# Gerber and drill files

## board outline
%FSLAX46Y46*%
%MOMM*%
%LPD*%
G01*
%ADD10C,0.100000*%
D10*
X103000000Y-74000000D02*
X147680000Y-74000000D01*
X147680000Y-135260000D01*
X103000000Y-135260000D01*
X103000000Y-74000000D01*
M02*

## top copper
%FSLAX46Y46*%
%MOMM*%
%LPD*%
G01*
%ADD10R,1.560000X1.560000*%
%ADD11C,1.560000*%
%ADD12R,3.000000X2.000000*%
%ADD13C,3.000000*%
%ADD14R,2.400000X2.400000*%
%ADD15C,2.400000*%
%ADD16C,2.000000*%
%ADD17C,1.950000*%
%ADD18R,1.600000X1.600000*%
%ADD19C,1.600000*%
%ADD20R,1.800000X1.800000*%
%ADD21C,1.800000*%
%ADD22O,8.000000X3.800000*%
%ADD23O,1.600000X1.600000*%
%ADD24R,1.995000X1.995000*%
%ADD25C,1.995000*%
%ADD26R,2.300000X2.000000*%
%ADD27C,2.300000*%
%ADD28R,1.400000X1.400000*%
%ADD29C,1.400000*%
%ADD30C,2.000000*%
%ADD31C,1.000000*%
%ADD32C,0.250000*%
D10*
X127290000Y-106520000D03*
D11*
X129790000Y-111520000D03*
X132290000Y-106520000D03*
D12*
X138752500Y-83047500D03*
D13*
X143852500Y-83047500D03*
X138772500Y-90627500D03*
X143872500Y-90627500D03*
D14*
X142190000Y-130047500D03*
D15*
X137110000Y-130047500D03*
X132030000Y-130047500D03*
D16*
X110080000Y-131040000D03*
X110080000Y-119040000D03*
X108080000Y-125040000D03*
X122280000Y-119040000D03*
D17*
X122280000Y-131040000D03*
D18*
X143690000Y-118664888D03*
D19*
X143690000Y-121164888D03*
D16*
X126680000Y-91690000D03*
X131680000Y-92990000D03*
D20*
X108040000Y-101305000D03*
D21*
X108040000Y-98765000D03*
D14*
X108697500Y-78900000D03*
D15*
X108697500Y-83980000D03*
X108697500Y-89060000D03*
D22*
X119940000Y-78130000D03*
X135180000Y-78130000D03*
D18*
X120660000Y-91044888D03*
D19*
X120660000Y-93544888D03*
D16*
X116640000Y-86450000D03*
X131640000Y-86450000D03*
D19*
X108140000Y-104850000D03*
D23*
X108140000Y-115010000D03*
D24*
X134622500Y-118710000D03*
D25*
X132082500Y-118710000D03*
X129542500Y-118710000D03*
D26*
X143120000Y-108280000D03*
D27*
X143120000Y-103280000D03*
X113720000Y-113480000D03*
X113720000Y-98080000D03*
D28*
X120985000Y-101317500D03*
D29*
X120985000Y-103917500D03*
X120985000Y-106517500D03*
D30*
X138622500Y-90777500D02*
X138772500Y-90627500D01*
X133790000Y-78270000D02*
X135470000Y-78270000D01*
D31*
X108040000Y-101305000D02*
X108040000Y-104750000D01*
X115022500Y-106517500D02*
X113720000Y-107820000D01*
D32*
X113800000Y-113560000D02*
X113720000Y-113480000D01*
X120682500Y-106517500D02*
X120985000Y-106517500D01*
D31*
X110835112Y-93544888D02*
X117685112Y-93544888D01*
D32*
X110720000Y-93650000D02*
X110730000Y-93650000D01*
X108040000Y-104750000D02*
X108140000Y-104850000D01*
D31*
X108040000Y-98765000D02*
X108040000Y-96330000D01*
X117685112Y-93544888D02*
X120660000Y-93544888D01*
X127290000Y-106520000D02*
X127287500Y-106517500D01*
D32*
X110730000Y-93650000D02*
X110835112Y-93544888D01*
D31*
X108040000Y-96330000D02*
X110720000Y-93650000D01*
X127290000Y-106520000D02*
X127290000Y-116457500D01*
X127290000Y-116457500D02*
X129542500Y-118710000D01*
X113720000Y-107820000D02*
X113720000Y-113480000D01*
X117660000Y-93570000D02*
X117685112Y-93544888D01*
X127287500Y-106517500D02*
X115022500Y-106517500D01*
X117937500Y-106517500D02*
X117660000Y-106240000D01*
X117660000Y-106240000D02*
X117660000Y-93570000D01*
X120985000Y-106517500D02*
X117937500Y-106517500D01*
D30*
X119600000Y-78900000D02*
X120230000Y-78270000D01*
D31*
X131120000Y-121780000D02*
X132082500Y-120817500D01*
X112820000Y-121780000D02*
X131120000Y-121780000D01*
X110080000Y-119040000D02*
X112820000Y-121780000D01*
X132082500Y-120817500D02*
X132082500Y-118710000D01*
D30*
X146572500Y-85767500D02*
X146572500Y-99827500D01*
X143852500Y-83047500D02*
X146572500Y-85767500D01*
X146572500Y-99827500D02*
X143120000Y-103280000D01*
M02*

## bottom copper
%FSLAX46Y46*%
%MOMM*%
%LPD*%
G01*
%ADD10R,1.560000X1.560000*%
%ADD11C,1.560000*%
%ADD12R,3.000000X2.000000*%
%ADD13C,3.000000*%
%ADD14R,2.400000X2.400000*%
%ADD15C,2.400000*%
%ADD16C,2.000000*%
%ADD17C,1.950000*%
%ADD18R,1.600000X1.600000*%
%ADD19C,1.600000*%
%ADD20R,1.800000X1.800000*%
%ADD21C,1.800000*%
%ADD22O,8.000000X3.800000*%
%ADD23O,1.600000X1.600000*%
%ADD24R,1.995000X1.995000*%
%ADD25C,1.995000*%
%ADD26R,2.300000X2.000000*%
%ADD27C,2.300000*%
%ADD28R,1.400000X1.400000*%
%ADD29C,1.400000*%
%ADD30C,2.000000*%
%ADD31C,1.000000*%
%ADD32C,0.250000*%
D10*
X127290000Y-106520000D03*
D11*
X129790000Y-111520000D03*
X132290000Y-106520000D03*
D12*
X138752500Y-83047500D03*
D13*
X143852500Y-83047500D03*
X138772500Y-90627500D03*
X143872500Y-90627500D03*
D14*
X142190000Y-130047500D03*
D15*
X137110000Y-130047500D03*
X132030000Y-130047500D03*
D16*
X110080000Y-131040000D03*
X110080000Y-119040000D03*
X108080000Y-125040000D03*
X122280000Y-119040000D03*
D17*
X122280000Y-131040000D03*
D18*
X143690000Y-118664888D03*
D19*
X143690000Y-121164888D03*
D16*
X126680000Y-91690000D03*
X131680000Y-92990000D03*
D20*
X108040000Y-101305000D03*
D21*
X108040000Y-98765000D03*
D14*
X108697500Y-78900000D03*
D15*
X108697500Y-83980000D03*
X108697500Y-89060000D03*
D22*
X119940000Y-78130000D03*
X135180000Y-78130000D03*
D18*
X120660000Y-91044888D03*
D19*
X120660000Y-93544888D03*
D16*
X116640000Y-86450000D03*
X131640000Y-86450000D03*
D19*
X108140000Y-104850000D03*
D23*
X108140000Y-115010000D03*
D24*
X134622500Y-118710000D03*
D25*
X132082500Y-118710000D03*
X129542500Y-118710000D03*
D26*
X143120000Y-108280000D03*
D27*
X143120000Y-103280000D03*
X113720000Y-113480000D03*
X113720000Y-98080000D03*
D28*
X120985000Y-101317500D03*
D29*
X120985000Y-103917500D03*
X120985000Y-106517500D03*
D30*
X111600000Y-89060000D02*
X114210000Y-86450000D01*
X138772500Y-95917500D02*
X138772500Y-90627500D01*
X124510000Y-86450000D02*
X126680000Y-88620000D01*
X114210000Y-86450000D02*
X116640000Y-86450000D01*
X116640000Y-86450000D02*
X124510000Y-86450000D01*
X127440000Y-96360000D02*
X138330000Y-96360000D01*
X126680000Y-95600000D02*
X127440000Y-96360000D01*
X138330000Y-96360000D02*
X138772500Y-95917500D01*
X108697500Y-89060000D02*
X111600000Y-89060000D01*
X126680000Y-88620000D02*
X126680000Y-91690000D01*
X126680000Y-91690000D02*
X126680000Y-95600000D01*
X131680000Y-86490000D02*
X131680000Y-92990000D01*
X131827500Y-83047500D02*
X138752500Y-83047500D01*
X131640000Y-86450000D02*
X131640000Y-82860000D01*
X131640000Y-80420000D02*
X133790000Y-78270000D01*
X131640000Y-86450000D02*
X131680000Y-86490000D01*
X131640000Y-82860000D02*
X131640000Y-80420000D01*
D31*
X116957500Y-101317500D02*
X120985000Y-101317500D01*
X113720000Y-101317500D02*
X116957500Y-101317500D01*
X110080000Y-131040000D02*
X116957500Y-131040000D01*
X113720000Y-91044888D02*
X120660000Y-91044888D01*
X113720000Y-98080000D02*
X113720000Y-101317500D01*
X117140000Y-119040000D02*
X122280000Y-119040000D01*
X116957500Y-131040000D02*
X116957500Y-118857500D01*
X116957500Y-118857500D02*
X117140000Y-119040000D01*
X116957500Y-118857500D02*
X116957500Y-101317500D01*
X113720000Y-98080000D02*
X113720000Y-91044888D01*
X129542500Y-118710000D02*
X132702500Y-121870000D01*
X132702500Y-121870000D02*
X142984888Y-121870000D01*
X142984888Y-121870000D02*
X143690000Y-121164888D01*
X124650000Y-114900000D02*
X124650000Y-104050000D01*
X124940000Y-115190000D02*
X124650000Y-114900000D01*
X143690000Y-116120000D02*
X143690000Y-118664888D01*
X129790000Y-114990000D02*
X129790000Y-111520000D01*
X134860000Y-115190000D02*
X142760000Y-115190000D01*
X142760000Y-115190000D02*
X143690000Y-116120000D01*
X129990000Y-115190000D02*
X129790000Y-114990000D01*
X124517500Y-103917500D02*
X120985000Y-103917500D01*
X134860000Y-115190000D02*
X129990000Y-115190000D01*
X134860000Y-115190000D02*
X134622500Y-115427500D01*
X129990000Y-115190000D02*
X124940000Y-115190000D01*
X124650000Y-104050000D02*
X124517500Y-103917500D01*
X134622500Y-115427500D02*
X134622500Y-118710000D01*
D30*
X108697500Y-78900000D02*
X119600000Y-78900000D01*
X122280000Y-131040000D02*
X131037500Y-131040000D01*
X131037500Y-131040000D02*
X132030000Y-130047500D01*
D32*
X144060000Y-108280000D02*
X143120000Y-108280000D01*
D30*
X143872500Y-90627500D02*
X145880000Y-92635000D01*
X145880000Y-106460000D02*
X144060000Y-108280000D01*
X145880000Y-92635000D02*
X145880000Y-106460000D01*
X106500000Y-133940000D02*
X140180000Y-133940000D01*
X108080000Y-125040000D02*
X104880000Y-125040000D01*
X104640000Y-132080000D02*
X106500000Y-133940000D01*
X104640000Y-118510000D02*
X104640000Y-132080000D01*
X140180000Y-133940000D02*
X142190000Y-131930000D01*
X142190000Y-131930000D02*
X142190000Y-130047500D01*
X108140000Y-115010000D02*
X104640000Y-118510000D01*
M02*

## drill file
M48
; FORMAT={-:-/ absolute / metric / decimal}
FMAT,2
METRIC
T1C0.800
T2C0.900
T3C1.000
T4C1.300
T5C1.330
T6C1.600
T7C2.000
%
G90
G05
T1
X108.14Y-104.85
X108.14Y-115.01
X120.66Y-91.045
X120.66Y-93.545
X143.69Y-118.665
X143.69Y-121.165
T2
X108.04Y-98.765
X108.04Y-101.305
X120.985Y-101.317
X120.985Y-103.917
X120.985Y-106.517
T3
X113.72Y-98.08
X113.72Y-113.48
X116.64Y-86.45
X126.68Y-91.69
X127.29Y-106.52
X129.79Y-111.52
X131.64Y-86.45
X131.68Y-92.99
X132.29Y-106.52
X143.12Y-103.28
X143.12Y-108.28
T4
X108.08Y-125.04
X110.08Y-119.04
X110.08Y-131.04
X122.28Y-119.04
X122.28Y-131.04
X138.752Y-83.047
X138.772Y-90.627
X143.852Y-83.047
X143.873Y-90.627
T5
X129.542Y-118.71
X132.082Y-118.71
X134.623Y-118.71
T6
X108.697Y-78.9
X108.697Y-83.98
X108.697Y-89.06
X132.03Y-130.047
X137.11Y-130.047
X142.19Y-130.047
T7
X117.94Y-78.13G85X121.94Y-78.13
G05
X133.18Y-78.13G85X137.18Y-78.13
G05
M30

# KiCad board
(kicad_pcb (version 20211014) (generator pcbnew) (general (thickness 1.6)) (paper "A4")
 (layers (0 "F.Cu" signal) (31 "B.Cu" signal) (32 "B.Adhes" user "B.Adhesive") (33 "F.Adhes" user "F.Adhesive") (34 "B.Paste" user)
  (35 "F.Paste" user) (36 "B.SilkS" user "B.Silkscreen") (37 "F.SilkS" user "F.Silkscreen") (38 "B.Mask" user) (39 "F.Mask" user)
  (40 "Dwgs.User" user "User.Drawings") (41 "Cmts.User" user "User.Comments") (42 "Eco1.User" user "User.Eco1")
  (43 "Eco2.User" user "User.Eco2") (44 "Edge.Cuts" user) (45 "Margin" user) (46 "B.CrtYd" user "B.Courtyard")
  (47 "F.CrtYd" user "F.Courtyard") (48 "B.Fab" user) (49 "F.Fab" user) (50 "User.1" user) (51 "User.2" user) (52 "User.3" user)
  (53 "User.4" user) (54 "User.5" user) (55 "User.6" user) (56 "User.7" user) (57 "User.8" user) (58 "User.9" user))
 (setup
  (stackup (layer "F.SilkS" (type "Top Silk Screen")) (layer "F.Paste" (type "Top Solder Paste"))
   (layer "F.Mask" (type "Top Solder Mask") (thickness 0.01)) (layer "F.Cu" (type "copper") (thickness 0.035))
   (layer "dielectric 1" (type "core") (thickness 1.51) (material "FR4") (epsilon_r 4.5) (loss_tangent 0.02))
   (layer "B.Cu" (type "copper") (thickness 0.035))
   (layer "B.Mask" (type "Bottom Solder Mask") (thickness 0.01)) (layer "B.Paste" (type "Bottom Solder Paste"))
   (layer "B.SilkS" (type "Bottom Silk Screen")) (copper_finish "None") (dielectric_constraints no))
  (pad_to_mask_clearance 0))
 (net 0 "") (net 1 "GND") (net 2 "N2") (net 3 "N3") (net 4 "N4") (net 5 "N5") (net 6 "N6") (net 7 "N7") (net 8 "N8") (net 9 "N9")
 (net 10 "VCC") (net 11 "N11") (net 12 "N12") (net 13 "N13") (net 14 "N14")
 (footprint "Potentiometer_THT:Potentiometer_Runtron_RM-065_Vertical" (layer "F.Cu") (at 127.29 106.52)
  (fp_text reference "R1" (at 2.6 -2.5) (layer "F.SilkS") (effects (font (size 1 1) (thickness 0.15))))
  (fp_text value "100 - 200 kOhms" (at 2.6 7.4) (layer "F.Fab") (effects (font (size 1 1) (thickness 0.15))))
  (pad "1" thru_hole rect (at 0 0) (size 1.56 1.56) (drill 1) (layers *.Cu *.Mask) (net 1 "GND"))
  (pad "2" thru_hole circle (at 2.5 5) (size 1.56 1.56) (drill 1) (layers *.Cu *.Mask) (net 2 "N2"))
  (pad "3" thru_hole circle (at 5 0) (size 1.56 1.56) (drill 1) (layers *.Cu *.Mask)))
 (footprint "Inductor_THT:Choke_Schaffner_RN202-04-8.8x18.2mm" (layer "F.Cu") (at 138.7725 75.4275)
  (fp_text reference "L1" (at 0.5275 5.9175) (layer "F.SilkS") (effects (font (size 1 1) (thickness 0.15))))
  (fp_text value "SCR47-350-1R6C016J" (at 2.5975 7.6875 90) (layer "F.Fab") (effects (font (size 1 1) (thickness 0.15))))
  (pad "1" thru_hole rect (at -0.02 7.62) (size 3 2) (drill 1.3) (layers *.Cu *.Mask) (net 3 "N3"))
  (pad "2" thru_hole circle (at 5.08 7.62) (size 3 3) (drill 1.3) (layers *.Cu *.Mask) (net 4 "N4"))
  (pad "3" thru_hole circle (at 0 15.2) (size 3 3) (drill 1.3) (layers *.Cu *.Mask) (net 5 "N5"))
  (pad "4" thru_hole circle (at 5.1 15.2) (size 3 3) (drill 1.3) (layers *.Cu *.Mask) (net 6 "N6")))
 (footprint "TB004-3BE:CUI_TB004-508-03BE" (layer "F.Cu") (at 142.19 130.0475 180)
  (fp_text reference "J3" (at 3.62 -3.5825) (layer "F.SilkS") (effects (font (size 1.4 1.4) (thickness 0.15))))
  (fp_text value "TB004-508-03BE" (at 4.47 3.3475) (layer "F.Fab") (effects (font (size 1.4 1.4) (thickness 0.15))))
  (pad "1" thru_hole rect locked (at 0 0 180) (size 2.4 2.4) (drill 1.6) (layers *.Cu *.Mask) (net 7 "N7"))
  (pad "2" thru_hole circle locked (at 5.08 0 180) (size 2.4 2.4) (drill 1.6) (layers *.Cu *.Mask) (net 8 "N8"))
  (pad "3" thru_hole circle locked (at 10.16 0 180) (size 2.4 2.4) (drill 1.6) (layers *.Cu *.Mask) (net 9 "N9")))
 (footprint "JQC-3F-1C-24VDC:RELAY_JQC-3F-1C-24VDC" (layer "F.Cu") (at 116.18 125.04 180)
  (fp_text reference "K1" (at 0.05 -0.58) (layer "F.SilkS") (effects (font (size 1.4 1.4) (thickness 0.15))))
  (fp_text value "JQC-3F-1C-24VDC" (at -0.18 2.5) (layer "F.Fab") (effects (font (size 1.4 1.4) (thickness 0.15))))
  (pad "COIL1" thru_hole circle locked (at 6.1 -6 180) (size 2 2) (drill 1.3) (layers *.Cu *.Mask) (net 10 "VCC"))
  (pad "COIL2" thru_hole circle locked (at 6.1 6 180) (size 2 2) (drill 1.3) (layers *.Cu *.Mask) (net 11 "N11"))
  (pad "COM" thru_hole circle locked (at 8.1 0 180) (size 2 2) (drill 1.3) (layers *.Cu *.Mask) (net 7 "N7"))
  (pad "NC" thru_hole circle locked (at -6.1 6 180) (size 2 2) (drill 1.3) (layers *.Cu *.Mask) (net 10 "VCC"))
  (pad "NO" thru_hole circle locked (at -6.1 -6 180) (size 1.95 1.95) (drill 1.3) (layers *.Cu *.Mask) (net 9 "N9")))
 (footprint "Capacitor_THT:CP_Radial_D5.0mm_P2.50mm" (layer "F.Cu") (at 143.69 118.664888 -90)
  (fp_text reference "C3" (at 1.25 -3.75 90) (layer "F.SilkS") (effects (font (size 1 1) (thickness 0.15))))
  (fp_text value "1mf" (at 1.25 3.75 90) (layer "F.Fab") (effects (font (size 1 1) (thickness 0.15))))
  (pad "1" thru_hole rect (at 0 0 270) (size 1.6 1.6) (drill 0.8) (layers *.Cu *.Mask) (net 2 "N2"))
  (pad "2" thru_hole circle (at 2.5 0 270) (size 1.6 1.6) (drill 0.8) (layers *.Cu *.Mask) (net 1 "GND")))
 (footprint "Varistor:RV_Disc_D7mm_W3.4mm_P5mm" (layer "F.Cu") (at 126.68 91.69)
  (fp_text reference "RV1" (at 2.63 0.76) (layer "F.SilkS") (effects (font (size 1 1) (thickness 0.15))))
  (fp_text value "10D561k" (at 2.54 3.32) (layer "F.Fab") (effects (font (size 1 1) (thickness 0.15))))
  (pad "1" thru_hole circle (at 0 0) (size 2 2) (drill 1) (layers *.Cu *.Mask) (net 5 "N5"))
  (pad "2" thru_hole circle (at 5 1.3) (size 2 2) (drill 1) (layers *.Cu *.Mask "F.Adhes") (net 3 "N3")))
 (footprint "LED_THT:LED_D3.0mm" (layer "F.Cu") (at 108.04 101.305 90)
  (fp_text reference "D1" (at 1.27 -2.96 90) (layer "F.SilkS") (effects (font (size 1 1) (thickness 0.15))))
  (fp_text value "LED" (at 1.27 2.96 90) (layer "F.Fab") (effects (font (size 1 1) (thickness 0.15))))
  (pad "1" thru_hole rect (at 0 0 90) (size 1.8 1.8) (drill 0.9) (layers *.Cu *.Mask) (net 1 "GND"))
  (pad "2" thru_hole circle (at 2.54 0 90) (size 1.8 1.8) (drill 0.9) (layers *.Cu *.Mask) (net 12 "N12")))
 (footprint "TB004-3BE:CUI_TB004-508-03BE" (layer "F.Cu") (at 108.6975 78.9 -90)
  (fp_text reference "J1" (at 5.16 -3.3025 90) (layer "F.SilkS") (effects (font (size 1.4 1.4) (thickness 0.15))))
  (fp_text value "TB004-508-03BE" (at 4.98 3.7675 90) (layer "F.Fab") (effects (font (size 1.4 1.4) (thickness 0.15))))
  (pad "1" thru_hole rect locked (at 0 0 270) (size 2.4 2.4) (drill 1.6) (layers *.Cu *.Mask) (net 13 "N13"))
  (pad "2" thru_hole circle locked (at 5.08 0 270) (size 2.4 2.4) (drill 1.6) (layers *.Cu *.Mask) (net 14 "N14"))
  (pad "3" thru_hole circle locked (at 10.16 0 270) (size 2.4 2.4) (drill 1.6) (layers *.Cu *.Mask) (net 5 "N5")))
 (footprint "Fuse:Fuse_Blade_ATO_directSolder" (layer "F.Cu") (at 122.48 78.13)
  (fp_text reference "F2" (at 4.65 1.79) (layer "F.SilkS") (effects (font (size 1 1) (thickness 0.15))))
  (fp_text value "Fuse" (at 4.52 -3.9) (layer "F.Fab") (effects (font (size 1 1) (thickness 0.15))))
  (pad "1" thru_hole oval (at -2.54 0) (size 8 3.8) (drill oval 6 2) (layers *.Cu *.Mask) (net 13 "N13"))
  (pad "2" thru_hole oval (at 12.7 0) (size 8 3.8) (drill oval 6 2) (layers *.Cu *.Mask) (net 3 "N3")))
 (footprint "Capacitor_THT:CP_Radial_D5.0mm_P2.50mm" (layer "F.Cu") (at 120.66 91.044888 -90)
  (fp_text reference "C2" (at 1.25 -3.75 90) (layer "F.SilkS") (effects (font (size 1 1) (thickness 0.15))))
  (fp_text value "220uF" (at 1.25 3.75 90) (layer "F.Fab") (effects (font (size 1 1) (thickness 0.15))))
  (pad "1" thru_hole rect (at 0 0 270) (size 1.6 1.6) (drill 0.8) (layers *.Cu *.Mask) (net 10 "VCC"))
  (pad "2" thru_hole circle (at 2.5 0 270) (size 1.6 1.6) (drill 0.8) (layers *.Cu *.Mask) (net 1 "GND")))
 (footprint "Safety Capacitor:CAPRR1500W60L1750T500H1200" (layer "F.Cu") (at 124.14 86.45)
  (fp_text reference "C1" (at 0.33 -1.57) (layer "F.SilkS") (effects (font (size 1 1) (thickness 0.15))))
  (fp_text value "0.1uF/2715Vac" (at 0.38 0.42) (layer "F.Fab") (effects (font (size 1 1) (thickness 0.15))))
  (pad "1" thru_hole circle locked (at -7.5 0) (size 2 2) (drill 1) (layers *.Cu *.Mask) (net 5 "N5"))
  (pad "2" thru_hole circle locked (at 7.5 0) (size 2 2) (drill 1) (layers *.Cu *.Mask) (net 3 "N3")))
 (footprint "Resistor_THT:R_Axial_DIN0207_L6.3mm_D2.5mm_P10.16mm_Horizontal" (layer "F.Cu") (at 108.14 104.85 -90)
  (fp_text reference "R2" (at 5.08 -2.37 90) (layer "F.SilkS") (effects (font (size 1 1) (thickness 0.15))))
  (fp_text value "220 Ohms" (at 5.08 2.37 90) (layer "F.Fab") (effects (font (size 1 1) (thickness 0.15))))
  (pad "1" thru_hole circle (at 0 0 270) (size 1.6 1.6) (drill 0.8) (layers *.Cu *.Mask) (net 12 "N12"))
  (pad "2" thru_hole oval (at 10.16 0 270) (size 1.6 1.6) (drill 0.8) (layers *.Cu *.Mask) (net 7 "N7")))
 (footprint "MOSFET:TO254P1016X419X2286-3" (layer "F.Cu") (at 132.0825 118.71 180)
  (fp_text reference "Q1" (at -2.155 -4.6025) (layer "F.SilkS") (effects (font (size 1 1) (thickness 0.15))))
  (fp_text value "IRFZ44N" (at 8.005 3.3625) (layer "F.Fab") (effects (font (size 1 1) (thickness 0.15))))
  (pad "1" thru_hole rect (at -2.54 0 180) (size 1.995 1.995) (drill 1.33) (layers *.Cu *.Mask) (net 2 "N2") (solder_mask_margin 0.102))
  (pad "2" thru_hole circle (at 0 0 180) (size 1.995 1.995) (drill 1.33) (layers *.Cu *.Mask) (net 11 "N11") (solder_mask_margin 0.102))
  (pad "3" thru_hole circle (at 2.54 0 180) (size 1.995 1.995) (drill 1.33) (layers *.Cu *.Mask) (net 1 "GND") (solder_mask_margin 0.102)))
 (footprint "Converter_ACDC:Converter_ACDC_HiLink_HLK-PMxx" (layer "F.Cu") (at 143.12 108.28 180)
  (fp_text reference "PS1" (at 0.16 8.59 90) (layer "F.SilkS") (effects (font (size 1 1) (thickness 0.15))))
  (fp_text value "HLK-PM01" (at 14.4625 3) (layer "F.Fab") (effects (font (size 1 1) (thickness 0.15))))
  (pad "1" thru_hole rect (at 0 0 180) (size 2.3 2) (drill 1) (layers *.Cu *.Mask) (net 6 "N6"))
  (pad "2" thru_hole circle (at 0 5 180) (size 2.3 2.3) (drill 1) (layers *.Cu *.Mask) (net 4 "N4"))
  (pad "3" thru_hole circle (at 29.4 -5.2 180) (size 2.3 2.3) (drill 1) (layers *.Cu *.Mask) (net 1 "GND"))
  (pad "4" thru_hole circle (at 29.4 10.2 180) (size 2.3 2.3) (drill 1) (layers *.Cu *.Mask) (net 10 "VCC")))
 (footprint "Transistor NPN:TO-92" (layer "B.Cu") (at 120.985 103.9175 -90)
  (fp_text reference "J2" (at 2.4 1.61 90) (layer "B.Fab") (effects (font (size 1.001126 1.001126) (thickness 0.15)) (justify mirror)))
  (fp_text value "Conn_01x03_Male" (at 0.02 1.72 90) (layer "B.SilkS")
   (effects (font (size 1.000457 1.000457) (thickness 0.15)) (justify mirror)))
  (pad "1" thru_hole rect locked (at -2.6 0 270) (size 1.4 1.4) (drill 0.9) (layers *.Cu *.Mask) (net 10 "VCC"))
  (pad "2" thru_hole circle locked (at 0 0 270) (size 1.4 1.4) (drill 0.9) (layers *.Cu *.Mask) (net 2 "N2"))
  (pad "3" thru_hole circle locked (at 2.6 0 270) (size 1.4 1.4) (drill 0.9) (layers *.Cu *.Mask) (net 1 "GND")))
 (gr_rect (start 103 74) (end 147.68 135.26) (layer "Edge.Cuts") (width 0.1) (fill none))
 (segment (start 138.6225 90.7775) (end 138.7725 90.6275) (width 2) (layer "F.Cu") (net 5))
 (segment (start 111.6 89.06) (end 114.21 86.45) (width 2) (layer "B.Cu") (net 5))
 (segment (start 138.7725 95.9175) (end 138.7725 90.6275) (width 2) (layer "B.Cu") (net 5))
 (segment (start 124.51 86.45) (end 126.68 88.62) (width 2) (layer "B.Cu") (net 5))
 (segment (start 114.21 86.45) (end 116.64 86.45) (width 2) (layer "B.Cu") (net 5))
 (segment (start 116.64 86.45) (end 124.51 86.45) (width 2) (layer "B.Cu") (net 5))
 (segment (start 127.44 96.36) (end 138.33 96.36) (width 2) (layer "B.Cu") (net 5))
 (segment (start 126.68 95.6) (end 127.44 96.36) (width 2) (layer "B.Cu") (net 5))
 (segment (start 138.33 96.36) (end 138.7725 95.9175) (width 2) (layer "B.Cu") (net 5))
 (segment (start 108.6975 89.06) (end 111.6 89.06) (width 2) (layer "B.Cu") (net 5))
 (segment (start 126.68 88.62) (end 126.68 91.69) (width 2) (layer "B.Cu") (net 5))
 (segment (start 126.68 91.69) (end 126.68 95.6) (width 2) (layer "B.Cu") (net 5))
 (segment (start 133.79 78.27) (end 135.47 78.27) (width 2) (layer "F.Cu") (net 3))
 (segment (start 131.68 86.49) (end 131.68 92.99) (width 2) (layer "B.Cu") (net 3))
 (segment (start 131.8275 83.0475) (end 138.7525 83.0475) (width 2) (layer "B.Cu") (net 3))
 (segment (start 131.64 86.45) (end 131.64 82.86) (width 2) (layer "B.Cu") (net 3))
 (segment (start 131.64 80.42) (end 133.79 78.27) (width 2) (layer "B.Cu") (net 3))
 (segment (start 131.64 86.45) (end 131.68 86.49) (width 2) (layer "B.Cu") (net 3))
 (segment (start 131.64 82.86) (end 131.64 80.42) (width 2) (layer "B.Cu") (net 3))
 (segment (start 116.9575 101.3175) (end 120.985 101.3175) (width 1) (layer "B.Cu") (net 10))
 (segment (start 113.72 101.3175) (end 116.9575 101.3175) (width 1) (layer "B.Cu") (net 10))
 (segment (start 110.08 131.04) (end 116.9575 131.04) (width 1) (layer "B.Cu") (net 10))
 (segment (start 113.72 91.044888) (end 120.66 91.044888) (width 1) (layer "B.Cu") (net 10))
 (segment (start 113.72 98.08) (end 113.72 101.3175) (width 1) (layer "B.Cu") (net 10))
 (segment (start 117.14 119.04) (end 122.28 119.04) (width 1) (layer "B.Cu") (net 10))
 (segment (start 116.9575 131.04) (end 116.9575 118.8575) (width 1) (layer "B.Cu") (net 10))
 (segment (start 116.9575 118.8575) (end 117.14 119.04) (width 1) (layer "B.Cu") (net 10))
 (segment (start 116.9575 118.8575) (end 116.9575 101.3175) (width 1) (layer "B.Cu") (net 10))
 (segment (start 113.72 98.08) (end 113.72 91.044888) (width 1) (layer "B.Cu") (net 10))
 (segment (start 108.04 101.305) (end 108.04 104.75) (width 1) (layer "F.Cu") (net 1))
 (segment (start 115.0225 106.5175) (end 113.72 107.82) (width 1) (layer "F.Cu") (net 1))
 (segment (start 113.8 113.56) (end 113.72 113.48) (width 0.25) (layer "F.Cu") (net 1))
 (segment (start 120.6825 106.5175) (end 120.985 106.5175) (width 0.25) (layer "F.Cu") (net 1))
 (segment (start 110.835112 93.544888) (end 117.685112 93.544888) (width 1) (layer "F.Cu") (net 1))
 (segment (start 110.72 93.65) (end 110.73 93.65) (width 0.25) (layer "F.Cu") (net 1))
 (segment (start 108.04 104.75) (end 108.14 104.85) (width 0.25) (layer "F.Cu") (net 1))
 (segment (start 108.04 98.765) (end 108.04 96.33) (width 1) (layer "F.Cu") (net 1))
 (segment (start 117.685112 93.544888) (end 120.66 93.544888) (width 1) (layer "F.Cu") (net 1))
 (segment (start 127.29 106.52) (end 127.2875 106.5175) (width 1) (layer "F.Cu") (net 1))
 (segment (start 110.73 93.65) (end 110.835112 93.544888) (width 0.25) (layer "F.Cu") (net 1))
 (segment (start 108.04 96.33) (end 110.72 93.65) (width 1) (layer "F.Cu") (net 1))
 (segment (start 127.29 106.52) (end 127.29 116.4575) (width 1) (layer "F.Cu") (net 1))
 (segment (start 127.29 116.4575) (end 129.5425 118.71) (width 1) (layer "F.Cu") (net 1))
 (segment (start 113.72 107.82) (end 113.72 113.48) (width 1) (layer "F.Cu") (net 1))
 (segment (start 117.66 93.57) (end 117.685112 93.544888) (width 1) (layer "F.Cu") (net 1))
 (segment (start 127.2875 106.5175) (end 115.0225 106.5175) (width 1) (layer "F.Cu") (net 1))
 (segment (start 117.9375 106.5175) (end 117.66 106.24) (width 1) (layer "F.Cu") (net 1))
 (segment (start 117.66 106.24) (end 117.66 93.57) (width 1) (layer "F.Cu") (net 1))
 (segment (start 120.985 106.5175) (end 117.9375 106.5175) (width 1) (layer "F.Cu") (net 1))
 (segment (start 129.5425 118.71) (end 132.7025 121.87) (width 1) (layer "B.Cu") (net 1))
 (segment (start 132.7025 121.87) (end 142.984888 121.87) (width 1) (layer "B.Cu") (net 1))
 (segment (start 142.984888 121.87) (end 143.69 121.164888) (width 1) (layer "B.Cu") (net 1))
 (segment (start 124.65 114.9) (end 124.65 104.05) (width 1) (layer "B.Cu") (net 2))
 (segment (start 124.94 115.19) (end 124.65 114.9) (width 1) (layer "B.Cu") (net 2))
 (segment (start 143.69 116.12) (end 143.69 118.664888) (width 1) (layer "B.Cu") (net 2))
 (segment (start 129.79 114.99) (end 129.79 111.52) (width 1) (layer "B.Cu") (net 2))
 (segment (start 134.86 115.19) (end 142.76 115.19) (width 1) (layer "B.Cu") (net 2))
 (segment (start 142.76 115.19) (end 143.69 116.12) (width 1) (layer "B.Cu") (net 2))
 (segment (start 129.99 115.19) (end 129.79 114.99) (width 1) (layer "B.Cu") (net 2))
 (segment (start 124.5175 103.9175) (end 120.985 103.9175) (width 1) (layer "B.Cu") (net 2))
 (segment (start 134.86 115.19) (end 129.99 115.19) (width 1) (layer "B.Cu") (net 2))
 (segment (start 134.86 115.19) (end 134.6225 115.4275) (width 1) (layer "B.Cu") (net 2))
 (segment (start 129.99 115.19) (end 124.94 115.19) (width 1) (layer "B.Cu") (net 2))
 (segment (start 124.65 104.05) (end 124.5175 103.9175) (width 1) (layer "B.Cu") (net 2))
 (segment (start 134.6225 115.4275) (end 134.6225 118.71) (width 1) (layer "B.Cu") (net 2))
 (segment (start 119.6 78.9) (end 120.23 78.27) (width 2) (layer "F.Cu") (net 13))
 (segment (start 108.6975 78.9) (end 119.6 78.9) (width 2) (layer "B.Cu") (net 13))
 (segment (start 122.28 131.04) (end 131.0375 131.04) (width 2) (layer "B.Cu") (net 9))
 (segment (start 131.0375 131.04) (end 132.03 130.0475) (width 2) (layer "B.Cu") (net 9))
 (segment (start 131.12 121.78) (end 132.0825 120.8175) (width 1) (layer "F.Cu") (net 11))
 (segment (start 112.82 121.78) (end 131.12 121.78) (width 1) (layer "F.Cu") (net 11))
 (segment (start 110.08 119.04) (end 112.82 121.78) (width 1) (layer "F.Cu") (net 11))
 (segment (start 132.0825 120.8175) (end 132.0825 118.71) (width 1) (layer "F.Cu") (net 11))
 (segment (start 146.5725 85.7675) (end 146.5725 99.8275) (width 2) (layer "F.Cu") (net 4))
 (segment (start 143.8525 83.0475) (end 146.5725 85.7675) (width 2) (layer "F.Cu") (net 4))
 (segment (start 146.5725 99.8275) (end 143.12 103.28) (width 2) (layer "F.Cu") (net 4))
 (segment (start 144.06 108.28) (end 143.12 108.28) (width 0.25) (layer "B.Cu") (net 6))
 (segment (start 143.8725 90.6275) (end 145.88 92.635) (width 2) (layer "B.Cu") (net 6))
 (segment (start 145.88 106.46) (end 144.06 108.28) (width 2) (layer "B.Cu") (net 6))
 (segment (start 145.88 92.635) (end 145.88 106.46) (width 2) (layer "B.Cu") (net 6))
 (segment (start 106.5 133.94) (end 140.18 133.94) (width 2) (layer "B.Cu") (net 7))
 (segment (start 108.08 125.04) (end 104.88 125.04) (width 2) (layer "B.Cu") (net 7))
 (segment (start 104.64 132.08) (end 106.5 133.94) (width 2) (layer "B.Cu") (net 7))
 (segment (start 104.64 118.51) (end 104.64 132.08) (width 2) (layer "B.Cu") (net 7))
 (segment (start 140.18 133.94) (end 142.19 131.93) (width 2) (layer "B.Cu") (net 7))
 (segment (start 142.19 131.93) (end 142.19 130.0475) (width 2) (layer "B.Cu") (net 7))
 (segment (start 108.14 115.01) (end 104.64 118.51) (width 2) (layer "B.Cu") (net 7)))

